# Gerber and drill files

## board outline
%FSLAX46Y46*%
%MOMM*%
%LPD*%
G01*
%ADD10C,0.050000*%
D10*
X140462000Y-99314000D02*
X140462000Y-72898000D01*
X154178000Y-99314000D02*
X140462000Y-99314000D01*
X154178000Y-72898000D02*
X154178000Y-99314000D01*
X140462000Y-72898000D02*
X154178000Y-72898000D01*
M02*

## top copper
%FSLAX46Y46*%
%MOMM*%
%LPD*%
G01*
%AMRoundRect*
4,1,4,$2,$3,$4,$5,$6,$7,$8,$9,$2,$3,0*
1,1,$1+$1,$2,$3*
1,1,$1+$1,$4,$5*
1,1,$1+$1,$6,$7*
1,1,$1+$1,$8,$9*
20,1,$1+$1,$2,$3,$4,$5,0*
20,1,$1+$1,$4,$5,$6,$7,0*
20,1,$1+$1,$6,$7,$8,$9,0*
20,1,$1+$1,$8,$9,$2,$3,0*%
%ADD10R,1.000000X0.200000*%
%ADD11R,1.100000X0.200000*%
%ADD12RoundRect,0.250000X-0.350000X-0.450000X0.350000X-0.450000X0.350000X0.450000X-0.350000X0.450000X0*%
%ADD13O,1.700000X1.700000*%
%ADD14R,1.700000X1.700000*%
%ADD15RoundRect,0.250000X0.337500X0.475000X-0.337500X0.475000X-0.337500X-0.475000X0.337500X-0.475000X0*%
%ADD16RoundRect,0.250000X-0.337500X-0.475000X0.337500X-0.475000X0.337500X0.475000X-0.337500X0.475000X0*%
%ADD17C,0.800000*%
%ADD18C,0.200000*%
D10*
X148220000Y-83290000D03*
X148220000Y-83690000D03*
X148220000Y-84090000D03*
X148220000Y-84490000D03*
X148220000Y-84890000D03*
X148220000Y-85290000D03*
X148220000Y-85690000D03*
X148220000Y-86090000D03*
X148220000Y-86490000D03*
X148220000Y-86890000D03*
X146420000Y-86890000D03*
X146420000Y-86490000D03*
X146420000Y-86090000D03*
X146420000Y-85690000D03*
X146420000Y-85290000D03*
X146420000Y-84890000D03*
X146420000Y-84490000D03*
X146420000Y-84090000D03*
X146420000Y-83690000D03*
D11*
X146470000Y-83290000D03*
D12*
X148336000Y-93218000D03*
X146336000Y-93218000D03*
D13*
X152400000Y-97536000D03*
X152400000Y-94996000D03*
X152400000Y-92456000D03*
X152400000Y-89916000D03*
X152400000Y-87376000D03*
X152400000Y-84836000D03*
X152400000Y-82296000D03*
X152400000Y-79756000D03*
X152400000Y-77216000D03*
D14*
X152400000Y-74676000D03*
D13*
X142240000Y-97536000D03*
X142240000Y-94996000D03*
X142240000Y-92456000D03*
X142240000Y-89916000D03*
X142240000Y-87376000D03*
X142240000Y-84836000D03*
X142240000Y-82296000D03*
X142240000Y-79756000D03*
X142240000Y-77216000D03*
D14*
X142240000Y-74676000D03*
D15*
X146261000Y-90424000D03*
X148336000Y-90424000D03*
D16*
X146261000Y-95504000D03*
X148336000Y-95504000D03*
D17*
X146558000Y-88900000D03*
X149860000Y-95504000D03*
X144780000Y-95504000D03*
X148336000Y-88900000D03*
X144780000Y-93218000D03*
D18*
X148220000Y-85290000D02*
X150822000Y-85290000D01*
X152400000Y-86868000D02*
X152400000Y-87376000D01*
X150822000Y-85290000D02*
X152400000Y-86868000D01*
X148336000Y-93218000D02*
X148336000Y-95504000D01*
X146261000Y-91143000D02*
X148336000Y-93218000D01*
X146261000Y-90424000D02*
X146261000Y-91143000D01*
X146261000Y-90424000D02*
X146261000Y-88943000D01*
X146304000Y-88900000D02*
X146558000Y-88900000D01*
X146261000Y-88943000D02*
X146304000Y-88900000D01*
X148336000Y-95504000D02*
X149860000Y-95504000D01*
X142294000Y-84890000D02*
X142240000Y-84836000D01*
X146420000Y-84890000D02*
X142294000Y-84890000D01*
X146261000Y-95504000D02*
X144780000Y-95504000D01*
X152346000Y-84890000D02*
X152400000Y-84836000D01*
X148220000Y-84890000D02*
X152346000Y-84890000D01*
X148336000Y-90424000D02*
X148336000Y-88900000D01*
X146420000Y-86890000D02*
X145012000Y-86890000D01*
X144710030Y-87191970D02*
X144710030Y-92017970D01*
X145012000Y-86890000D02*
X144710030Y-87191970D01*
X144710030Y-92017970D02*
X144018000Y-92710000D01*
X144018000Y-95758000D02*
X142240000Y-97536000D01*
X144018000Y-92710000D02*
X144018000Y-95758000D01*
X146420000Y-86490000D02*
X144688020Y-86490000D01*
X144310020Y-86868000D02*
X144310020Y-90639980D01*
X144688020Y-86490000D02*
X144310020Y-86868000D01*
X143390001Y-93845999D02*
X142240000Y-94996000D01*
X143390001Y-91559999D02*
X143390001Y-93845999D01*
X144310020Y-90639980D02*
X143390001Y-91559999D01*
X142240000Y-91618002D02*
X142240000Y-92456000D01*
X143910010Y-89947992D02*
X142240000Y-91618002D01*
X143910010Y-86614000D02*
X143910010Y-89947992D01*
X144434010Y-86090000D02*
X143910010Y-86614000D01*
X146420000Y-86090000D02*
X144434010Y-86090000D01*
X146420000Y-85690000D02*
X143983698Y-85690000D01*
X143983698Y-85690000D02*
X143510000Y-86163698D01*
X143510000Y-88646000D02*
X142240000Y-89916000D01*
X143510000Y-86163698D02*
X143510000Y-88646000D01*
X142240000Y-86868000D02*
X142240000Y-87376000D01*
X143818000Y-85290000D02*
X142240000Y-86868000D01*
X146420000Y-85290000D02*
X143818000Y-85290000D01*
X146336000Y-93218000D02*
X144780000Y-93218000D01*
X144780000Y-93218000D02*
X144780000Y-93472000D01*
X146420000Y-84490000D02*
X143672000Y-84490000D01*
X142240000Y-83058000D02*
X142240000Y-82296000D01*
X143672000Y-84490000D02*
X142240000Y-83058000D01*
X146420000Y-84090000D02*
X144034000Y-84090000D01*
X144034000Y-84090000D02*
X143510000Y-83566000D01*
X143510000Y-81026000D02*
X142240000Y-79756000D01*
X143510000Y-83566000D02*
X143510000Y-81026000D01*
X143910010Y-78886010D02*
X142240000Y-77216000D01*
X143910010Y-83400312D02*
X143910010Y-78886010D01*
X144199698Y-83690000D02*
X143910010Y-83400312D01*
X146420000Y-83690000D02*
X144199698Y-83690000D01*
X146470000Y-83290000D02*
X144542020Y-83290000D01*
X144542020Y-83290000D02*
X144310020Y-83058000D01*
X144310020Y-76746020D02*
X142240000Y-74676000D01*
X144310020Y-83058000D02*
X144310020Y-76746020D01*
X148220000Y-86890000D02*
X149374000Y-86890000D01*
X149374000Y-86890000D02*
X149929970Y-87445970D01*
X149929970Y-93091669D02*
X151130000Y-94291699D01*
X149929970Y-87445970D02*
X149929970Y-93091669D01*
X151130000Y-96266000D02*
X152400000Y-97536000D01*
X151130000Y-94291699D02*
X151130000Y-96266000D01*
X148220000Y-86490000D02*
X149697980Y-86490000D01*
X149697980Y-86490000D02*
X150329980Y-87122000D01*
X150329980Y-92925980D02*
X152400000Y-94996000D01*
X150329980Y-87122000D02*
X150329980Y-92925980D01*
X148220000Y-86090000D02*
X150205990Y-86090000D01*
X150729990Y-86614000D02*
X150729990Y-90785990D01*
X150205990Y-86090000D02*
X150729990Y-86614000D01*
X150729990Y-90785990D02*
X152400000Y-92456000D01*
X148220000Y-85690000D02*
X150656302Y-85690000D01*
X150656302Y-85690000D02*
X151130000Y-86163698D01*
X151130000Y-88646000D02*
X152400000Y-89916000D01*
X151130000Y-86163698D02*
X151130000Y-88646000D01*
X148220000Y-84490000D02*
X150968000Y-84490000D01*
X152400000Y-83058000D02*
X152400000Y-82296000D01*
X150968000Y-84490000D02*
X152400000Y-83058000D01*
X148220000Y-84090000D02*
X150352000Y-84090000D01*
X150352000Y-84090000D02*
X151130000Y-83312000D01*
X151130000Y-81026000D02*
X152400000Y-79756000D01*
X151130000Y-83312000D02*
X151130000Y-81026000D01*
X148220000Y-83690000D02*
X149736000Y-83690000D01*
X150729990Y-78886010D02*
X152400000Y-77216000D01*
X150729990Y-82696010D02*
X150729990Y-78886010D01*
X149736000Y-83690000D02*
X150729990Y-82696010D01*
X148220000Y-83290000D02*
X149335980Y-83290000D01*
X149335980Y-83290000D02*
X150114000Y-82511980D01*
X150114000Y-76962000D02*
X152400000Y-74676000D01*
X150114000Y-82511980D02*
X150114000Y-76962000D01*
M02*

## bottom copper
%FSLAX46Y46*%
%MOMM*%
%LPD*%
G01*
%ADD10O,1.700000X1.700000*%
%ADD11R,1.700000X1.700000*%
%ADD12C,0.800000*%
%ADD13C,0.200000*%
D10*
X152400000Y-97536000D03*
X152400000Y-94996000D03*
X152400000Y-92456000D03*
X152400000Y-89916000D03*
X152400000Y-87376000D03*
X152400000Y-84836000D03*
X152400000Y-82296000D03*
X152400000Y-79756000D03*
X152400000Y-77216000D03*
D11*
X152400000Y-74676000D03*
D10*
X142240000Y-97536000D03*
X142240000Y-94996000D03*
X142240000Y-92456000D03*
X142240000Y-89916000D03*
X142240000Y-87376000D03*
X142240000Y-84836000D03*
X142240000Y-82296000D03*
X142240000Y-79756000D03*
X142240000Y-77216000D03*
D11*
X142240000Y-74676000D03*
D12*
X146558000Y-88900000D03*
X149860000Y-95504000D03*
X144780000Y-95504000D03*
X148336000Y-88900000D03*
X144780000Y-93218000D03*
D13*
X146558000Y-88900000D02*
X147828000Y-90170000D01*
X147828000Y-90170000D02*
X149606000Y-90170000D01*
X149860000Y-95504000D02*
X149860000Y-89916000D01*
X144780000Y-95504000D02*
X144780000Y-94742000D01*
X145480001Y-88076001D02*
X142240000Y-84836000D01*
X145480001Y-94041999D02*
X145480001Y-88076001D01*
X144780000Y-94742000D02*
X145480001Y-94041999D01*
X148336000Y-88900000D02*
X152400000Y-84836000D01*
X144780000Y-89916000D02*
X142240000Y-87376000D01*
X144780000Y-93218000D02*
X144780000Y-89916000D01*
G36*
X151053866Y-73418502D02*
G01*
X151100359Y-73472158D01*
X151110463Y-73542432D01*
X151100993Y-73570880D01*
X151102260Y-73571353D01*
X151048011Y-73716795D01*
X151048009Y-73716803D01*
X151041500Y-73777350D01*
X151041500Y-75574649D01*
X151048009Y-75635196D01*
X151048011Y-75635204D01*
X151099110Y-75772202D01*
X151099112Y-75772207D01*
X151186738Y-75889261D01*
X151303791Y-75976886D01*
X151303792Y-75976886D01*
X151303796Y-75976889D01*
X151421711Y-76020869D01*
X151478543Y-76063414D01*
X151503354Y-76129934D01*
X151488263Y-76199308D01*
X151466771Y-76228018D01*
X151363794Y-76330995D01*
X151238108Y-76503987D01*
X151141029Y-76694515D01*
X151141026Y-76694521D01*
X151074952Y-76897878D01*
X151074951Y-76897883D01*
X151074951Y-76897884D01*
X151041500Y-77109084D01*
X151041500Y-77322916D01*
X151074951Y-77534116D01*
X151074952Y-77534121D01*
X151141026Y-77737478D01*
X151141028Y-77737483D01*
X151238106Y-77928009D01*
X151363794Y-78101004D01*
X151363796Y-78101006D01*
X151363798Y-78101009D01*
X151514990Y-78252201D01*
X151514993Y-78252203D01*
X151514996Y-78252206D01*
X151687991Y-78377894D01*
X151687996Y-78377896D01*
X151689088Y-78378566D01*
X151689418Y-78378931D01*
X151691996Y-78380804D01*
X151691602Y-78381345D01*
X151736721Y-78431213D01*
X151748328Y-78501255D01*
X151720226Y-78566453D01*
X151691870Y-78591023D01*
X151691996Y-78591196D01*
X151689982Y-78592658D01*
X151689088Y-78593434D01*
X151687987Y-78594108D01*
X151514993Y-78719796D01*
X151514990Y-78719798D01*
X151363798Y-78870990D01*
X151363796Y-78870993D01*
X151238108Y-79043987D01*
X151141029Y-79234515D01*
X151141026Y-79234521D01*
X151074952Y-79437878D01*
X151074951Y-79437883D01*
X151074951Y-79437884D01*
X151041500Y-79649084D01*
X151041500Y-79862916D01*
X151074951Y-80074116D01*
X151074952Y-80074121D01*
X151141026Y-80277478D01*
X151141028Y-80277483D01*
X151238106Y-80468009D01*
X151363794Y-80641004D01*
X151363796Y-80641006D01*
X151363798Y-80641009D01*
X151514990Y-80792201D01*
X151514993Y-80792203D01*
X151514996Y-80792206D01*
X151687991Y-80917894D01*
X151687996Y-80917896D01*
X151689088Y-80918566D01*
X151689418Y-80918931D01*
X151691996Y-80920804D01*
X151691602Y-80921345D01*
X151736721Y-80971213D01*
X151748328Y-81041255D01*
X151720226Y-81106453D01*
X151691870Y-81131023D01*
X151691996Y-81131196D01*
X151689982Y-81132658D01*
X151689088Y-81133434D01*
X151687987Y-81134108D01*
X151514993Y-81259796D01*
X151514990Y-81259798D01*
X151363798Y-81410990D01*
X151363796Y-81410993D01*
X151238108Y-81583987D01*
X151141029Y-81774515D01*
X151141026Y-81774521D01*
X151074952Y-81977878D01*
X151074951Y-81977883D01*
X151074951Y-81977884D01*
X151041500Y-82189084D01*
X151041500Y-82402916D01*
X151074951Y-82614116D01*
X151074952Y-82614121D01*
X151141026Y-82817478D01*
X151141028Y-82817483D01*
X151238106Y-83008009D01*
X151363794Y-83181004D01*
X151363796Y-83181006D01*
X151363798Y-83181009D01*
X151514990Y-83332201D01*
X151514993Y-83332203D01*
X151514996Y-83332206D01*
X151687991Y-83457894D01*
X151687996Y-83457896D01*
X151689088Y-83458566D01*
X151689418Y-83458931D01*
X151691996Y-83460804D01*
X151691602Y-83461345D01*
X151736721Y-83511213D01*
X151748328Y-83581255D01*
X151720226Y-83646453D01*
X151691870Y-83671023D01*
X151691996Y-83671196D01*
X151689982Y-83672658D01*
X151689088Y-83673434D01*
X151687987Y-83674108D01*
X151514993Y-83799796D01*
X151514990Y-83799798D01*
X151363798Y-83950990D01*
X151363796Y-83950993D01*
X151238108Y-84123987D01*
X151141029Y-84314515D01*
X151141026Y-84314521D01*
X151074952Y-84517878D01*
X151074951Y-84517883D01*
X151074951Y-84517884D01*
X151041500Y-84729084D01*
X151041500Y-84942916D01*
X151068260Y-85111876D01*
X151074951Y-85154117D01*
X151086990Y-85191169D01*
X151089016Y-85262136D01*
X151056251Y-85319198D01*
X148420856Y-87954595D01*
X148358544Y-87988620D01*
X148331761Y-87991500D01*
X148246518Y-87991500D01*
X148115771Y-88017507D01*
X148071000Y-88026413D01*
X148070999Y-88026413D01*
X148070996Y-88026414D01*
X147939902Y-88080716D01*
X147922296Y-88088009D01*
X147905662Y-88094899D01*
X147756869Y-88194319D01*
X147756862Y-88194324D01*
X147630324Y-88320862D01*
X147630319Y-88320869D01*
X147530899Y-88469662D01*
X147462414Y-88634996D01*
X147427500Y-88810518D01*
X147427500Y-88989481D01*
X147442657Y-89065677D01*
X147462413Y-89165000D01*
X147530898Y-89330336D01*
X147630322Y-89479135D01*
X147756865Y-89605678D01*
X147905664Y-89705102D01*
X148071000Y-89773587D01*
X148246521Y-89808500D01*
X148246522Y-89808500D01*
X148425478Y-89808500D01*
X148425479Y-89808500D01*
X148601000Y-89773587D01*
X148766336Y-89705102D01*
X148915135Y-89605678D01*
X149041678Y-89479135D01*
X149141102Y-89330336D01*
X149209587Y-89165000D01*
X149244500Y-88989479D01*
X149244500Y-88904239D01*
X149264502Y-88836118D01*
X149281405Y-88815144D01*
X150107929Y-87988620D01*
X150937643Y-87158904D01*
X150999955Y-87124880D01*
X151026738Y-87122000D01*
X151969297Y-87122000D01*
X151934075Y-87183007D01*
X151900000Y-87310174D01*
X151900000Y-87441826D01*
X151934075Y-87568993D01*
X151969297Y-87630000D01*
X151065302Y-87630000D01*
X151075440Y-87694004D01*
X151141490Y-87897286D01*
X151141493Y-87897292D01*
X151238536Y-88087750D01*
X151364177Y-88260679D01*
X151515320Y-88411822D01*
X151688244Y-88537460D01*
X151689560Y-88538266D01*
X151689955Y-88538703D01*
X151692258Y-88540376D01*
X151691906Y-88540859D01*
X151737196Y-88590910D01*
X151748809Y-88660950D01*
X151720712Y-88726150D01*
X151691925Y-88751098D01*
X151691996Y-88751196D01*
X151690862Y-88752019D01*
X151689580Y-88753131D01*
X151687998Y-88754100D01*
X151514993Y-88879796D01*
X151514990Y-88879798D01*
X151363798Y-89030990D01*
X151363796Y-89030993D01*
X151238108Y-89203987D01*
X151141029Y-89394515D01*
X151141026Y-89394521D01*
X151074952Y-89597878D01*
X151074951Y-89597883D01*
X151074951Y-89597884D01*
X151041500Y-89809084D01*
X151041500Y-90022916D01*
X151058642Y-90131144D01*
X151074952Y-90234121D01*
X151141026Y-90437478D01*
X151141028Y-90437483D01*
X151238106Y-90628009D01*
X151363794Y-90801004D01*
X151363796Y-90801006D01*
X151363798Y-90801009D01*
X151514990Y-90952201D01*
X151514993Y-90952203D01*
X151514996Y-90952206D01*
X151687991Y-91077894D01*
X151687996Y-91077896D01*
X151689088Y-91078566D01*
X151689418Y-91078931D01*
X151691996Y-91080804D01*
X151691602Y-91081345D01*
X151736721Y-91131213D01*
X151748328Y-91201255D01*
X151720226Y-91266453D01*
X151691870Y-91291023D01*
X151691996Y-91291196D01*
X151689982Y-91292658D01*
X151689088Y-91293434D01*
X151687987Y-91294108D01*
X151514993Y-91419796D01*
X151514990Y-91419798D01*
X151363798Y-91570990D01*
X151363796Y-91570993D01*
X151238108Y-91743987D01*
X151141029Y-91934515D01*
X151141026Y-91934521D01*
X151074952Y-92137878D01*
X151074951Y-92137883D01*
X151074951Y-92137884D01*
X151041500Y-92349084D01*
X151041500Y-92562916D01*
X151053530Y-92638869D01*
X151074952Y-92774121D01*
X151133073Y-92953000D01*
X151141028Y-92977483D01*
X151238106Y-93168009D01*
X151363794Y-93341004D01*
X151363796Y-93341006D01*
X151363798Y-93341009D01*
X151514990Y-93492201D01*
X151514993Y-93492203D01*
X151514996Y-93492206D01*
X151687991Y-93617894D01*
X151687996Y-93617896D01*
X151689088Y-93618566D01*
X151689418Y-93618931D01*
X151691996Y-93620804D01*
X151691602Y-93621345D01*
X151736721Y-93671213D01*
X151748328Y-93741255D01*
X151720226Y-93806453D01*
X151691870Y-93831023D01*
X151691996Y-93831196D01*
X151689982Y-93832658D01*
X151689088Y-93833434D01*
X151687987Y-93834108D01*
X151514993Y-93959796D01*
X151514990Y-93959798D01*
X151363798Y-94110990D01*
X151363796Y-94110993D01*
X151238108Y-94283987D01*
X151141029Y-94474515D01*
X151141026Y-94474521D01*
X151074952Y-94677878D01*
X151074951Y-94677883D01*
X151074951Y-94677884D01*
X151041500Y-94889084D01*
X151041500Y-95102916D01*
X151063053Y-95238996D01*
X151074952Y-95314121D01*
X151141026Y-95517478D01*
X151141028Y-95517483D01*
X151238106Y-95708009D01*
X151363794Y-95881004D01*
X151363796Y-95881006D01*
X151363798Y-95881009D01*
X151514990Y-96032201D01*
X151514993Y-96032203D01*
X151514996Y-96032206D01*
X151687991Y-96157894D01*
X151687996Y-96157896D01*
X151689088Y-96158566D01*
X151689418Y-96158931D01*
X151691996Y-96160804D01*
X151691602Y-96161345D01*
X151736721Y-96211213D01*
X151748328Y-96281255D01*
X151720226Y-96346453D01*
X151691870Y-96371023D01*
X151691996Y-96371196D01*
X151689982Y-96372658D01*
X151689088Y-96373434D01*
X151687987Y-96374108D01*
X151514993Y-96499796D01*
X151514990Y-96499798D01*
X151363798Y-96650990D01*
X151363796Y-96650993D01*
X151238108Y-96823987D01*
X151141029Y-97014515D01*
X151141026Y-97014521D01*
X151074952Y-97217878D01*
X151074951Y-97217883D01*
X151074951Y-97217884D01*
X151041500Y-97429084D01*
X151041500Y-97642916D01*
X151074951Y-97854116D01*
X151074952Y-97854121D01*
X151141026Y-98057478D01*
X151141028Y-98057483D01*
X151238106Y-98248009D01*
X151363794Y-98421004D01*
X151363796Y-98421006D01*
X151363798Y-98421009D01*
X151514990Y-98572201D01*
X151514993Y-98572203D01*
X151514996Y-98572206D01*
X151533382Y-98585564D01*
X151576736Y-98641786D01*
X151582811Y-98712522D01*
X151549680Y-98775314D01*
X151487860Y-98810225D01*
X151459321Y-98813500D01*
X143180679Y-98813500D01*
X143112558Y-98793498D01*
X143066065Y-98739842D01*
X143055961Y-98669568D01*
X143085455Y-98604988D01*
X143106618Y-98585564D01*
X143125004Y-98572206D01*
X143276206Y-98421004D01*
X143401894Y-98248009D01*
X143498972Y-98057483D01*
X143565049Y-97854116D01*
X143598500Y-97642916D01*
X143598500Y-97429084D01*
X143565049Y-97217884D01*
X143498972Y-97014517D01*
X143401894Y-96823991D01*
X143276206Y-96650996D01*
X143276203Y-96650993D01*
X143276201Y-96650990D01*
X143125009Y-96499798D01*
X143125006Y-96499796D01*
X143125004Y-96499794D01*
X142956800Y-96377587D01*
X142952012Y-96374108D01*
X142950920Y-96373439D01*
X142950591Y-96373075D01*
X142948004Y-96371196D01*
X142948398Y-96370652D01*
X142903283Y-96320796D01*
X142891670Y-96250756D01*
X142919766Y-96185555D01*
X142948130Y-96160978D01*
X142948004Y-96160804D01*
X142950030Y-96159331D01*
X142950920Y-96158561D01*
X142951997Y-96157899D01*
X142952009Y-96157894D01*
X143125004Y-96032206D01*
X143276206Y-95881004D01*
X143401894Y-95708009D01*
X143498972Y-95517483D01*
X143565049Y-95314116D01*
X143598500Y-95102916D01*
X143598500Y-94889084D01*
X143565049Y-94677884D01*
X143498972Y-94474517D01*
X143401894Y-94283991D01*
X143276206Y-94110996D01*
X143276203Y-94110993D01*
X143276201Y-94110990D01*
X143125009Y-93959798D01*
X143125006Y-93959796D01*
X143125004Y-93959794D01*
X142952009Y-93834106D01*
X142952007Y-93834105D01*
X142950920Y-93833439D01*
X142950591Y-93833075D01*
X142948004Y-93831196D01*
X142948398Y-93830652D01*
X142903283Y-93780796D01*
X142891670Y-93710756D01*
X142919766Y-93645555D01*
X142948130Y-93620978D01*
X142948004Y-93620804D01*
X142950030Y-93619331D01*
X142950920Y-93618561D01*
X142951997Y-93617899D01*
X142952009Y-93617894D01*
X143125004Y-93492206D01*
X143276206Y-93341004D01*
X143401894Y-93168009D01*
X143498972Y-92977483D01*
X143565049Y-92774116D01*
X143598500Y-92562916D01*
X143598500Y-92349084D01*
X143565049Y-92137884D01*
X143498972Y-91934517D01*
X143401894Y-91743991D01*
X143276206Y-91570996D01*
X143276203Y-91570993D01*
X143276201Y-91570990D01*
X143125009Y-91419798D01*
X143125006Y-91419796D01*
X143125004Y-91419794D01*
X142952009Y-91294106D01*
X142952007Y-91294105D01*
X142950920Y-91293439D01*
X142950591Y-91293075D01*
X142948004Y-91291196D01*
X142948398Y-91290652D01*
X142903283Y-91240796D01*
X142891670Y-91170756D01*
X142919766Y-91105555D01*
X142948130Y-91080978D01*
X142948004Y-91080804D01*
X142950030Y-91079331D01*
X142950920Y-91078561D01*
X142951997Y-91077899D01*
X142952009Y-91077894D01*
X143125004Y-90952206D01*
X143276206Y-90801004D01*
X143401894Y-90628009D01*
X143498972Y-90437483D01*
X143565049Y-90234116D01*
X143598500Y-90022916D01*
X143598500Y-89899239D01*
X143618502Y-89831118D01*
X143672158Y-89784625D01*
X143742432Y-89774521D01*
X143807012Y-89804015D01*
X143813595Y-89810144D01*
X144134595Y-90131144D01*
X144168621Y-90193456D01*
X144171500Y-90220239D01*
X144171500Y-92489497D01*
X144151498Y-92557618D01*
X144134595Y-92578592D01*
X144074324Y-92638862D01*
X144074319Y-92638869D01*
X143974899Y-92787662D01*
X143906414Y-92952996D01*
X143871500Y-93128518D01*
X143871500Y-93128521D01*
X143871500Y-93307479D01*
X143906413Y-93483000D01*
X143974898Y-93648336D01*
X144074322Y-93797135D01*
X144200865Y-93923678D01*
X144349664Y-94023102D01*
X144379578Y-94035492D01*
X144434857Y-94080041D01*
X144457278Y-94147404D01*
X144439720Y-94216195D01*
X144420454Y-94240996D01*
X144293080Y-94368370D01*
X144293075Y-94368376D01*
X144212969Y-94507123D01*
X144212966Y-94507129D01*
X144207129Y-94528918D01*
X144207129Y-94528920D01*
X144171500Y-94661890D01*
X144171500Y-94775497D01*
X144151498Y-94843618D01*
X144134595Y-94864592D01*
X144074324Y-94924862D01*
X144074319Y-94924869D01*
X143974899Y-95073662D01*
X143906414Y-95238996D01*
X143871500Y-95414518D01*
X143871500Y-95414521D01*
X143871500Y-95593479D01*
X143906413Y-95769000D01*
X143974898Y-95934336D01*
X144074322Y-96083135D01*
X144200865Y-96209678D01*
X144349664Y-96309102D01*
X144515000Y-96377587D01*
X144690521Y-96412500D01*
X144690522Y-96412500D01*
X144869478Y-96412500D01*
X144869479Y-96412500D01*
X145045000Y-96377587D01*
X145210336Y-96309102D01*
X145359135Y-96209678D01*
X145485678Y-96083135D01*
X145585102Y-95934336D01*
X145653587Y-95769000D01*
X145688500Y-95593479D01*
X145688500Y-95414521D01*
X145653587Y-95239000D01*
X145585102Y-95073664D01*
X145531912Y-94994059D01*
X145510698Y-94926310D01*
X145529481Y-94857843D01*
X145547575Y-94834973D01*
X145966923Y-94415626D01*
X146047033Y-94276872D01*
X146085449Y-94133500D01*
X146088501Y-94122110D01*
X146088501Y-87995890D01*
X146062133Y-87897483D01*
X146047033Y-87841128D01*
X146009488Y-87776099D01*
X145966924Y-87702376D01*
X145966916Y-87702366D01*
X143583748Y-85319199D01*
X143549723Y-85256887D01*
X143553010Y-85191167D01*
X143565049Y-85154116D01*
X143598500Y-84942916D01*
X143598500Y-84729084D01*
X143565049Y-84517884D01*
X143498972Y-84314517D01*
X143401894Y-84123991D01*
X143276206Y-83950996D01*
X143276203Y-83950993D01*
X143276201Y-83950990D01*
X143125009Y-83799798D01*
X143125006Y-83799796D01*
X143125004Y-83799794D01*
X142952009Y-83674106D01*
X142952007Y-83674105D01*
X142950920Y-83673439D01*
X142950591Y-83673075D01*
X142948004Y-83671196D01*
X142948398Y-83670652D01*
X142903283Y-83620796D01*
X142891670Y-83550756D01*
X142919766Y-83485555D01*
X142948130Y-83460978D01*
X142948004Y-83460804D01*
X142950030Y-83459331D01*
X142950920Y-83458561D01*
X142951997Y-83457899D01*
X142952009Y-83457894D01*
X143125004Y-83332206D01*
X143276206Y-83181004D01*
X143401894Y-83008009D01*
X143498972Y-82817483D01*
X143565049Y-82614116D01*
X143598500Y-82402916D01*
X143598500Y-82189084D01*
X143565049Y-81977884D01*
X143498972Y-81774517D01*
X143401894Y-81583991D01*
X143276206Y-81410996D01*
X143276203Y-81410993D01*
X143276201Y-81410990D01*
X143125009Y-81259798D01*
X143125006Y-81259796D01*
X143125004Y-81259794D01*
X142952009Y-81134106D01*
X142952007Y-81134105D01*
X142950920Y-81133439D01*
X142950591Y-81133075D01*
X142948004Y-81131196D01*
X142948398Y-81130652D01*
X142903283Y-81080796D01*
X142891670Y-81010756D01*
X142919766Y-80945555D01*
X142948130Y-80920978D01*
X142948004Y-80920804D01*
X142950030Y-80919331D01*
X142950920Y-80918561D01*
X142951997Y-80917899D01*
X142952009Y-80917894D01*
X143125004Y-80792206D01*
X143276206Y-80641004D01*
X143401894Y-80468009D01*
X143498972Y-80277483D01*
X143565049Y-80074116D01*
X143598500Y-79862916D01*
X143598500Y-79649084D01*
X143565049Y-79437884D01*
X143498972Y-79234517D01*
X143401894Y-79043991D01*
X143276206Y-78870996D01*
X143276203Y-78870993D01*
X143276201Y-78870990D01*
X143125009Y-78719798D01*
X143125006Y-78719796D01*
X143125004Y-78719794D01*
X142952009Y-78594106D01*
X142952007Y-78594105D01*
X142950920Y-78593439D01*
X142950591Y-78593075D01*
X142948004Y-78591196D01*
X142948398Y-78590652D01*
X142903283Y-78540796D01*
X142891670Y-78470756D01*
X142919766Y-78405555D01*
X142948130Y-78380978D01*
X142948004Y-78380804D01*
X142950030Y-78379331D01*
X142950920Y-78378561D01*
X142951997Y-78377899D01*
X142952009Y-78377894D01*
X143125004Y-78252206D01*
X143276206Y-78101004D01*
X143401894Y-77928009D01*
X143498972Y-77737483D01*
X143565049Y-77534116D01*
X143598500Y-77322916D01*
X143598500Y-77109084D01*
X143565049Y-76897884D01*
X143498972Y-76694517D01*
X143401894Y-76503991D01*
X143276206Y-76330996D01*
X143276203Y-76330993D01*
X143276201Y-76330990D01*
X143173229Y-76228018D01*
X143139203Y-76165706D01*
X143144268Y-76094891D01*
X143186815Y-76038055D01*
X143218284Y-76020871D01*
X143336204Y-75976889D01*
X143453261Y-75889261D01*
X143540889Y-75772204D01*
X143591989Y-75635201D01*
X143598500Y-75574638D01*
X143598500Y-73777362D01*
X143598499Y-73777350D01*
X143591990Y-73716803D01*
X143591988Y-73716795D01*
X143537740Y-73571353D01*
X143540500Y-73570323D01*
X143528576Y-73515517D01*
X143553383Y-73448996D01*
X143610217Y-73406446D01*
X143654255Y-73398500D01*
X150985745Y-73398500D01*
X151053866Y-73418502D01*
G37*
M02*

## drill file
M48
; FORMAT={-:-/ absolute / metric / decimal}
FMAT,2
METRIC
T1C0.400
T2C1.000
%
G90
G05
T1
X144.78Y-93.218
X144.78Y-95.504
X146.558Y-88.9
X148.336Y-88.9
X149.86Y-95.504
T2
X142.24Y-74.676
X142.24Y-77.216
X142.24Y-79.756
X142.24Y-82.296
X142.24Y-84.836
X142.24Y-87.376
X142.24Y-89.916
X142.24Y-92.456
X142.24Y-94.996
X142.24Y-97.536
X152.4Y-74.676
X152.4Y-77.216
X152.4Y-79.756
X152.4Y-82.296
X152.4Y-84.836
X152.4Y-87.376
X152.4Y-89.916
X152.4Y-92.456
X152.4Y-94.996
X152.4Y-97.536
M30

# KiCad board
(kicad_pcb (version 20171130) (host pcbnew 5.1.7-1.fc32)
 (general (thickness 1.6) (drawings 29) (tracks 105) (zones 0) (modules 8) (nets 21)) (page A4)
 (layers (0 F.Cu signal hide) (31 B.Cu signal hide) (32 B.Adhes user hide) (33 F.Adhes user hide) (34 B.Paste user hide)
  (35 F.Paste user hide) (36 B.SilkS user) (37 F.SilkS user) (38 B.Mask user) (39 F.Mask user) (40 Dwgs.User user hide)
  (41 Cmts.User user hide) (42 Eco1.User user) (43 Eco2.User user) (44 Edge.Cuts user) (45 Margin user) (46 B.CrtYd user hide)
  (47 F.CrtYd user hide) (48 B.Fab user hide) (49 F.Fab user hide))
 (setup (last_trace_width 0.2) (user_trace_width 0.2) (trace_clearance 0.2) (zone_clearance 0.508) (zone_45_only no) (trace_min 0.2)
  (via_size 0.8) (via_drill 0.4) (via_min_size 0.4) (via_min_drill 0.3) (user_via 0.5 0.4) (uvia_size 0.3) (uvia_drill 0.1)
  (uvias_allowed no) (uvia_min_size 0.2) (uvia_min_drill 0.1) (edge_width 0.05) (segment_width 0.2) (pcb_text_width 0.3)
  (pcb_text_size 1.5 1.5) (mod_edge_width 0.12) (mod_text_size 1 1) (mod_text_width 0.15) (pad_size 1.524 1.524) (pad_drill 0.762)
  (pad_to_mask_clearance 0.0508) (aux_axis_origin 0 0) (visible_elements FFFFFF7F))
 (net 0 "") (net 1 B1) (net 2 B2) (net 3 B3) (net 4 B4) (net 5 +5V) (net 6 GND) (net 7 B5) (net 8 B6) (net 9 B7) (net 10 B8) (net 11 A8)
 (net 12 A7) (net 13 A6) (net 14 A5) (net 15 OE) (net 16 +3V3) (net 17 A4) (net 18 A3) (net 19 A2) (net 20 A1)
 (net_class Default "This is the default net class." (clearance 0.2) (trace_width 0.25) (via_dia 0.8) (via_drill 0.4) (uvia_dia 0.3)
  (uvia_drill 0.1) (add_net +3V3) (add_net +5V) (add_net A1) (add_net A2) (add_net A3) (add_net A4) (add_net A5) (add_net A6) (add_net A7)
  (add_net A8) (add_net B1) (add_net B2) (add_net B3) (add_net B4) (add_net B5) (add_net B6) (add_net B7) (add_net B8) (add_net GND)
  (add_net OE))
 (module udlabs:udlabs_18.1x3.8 (layer B.Cu) (at 147.5232 85.598 90)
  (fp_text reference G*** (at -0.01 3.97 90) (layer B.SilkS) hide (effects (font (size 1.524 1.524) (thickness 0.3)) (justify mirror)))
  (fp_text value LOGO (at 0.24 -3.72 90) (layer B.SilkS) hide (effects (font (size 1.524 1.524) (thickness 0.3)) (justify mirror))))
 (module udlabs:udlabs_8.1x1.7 (layer F.Cu) (at 147.066 77.7494 90)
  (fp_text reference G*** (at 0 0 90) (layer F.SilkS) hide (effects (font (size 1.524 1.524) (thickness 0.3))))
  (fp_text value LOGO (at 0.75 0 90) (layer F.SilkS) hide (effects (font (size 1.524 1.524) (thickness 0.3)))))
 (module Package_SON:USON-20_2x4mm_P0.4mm (layer F.Cu) (at 147.32 85.09)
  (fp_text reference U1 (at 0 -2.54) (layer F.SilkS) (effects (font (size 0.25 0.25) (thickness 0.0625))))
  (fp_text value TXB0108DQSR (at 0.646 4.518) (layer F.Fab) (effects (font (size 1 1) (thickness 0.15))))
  (pad 20 smd rect (at 0.9 -1.8 270) (size 0.2 1) (layers F.Cu F.Paste F.Mask) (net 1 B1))
  (pad 19 smd rect (at 0.9 -1.4 270) (size 0.2 1) (layers F.Cu F.Paste F.Mask) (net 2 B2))
  (pad 18 smd rect (at 0.9 -1 270) (size 0.2 1) (layers F.Cu F.Paste F.Mask) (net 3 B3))
  (pad 17 smd rect (at 0.9 -0.6 270) (size 0.2 1) (layers F.Cu F.Paste F.Mask) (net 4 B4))
  (pad 16 smd rect (at 0.9 -0.2 270) (size 0.2 1) (layers F.Cu F.Paste F.Mask) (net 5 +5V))
  (pad 15 smd rect (at 0.9 0.2 270) (size 0.2 1) (layers F.Cu F.Paste F.Mask) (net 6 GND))
  (pad 14 smd rect (at 0.9 0.6 270) (size 0.2 1) (layers F.Cu F.Paste F.Mask) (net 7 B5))
  (pad 13 smd rect (at 0.9 1 270) (size 0.2 1) (layers F.Cu F.Paste F.Mask) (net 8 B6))
  (pad 12 smd rect (at 0.9 1.4 270) (size 0.2 1) (layers F.Cu F.Paste F.Mask) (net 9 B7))
  (pad 11 smd rect (at 0.9 1.8 270) (size 0.2 1) (layers F.Cu F.Paste F.Mask) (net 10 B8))
  (pad 10 smd rect (at -0.9 1.8 270) (size 0.2 1) (layers F.Cu F.Paste F.Mask) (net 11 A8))
  (pad 9 smd rect (at -0.9 1.4 270) (size 0.2 1) (layers F.Cu F.Paste F.Mask) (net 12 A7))
  (pad 8 smd rect (at -0.9 1 270) (size 0.2 1) (layers F.Cu F.Paste F.Mask) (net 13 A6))
  (pad 7 smd rect (at -0.9 0.6 270) (size 0.2 1) (layers F.Cu F.Paste F.Mask) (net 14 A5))
  (pad 6 smd rect (at -0.9 0.2 270) (size 0.2 1) (layers F.Cu F.Paste F.Mask) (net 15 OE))
  (pad 5 smd rect (at -0.9 -0.2 270) (size 0.2 1) (layers F.Cu F.Paste F.Mask) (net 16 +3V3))
  (pad 4 smd rect (at -0.9 -0.6 270) (size 0.2 1) (layers F.Cu F.Paste F.Mask) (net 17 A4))
  (pad 3 smd rect (at -0.9 -1 270) (size 0.2 1) (layers F.Cu F.Paste F.Mask) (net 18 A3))
  (pad 2 smd rect (at -0.9 -1.4 270) (size 0.2 1) (layers F.Cu F.Paste F.Mask) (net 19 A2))
  (pad 1 smd rect (at -0.85 -1.8 270) (size 0.2 1.1) (layers F.Cu F.Paste F.Mask) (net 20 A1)))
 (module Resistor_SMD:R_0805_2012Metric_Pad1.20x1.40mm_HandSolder (layer F.Cu) (at 147.336 93.218)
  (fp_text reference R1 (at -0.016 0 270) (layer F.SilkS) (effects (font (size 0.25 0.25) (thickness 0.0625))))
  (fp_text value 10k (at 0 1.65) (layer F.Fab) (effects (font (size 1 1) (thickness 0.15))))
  (pad 2 smd roundrect (at 1 0) (size 1.2 1.4) (layers F.Cu F.Paste F.Mask) (roundrect_rratio 0.208333) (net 6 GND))
  (pad 1 smd roundrect (at -1 0) (size 1.2 1.4) (layers F.Cu F.Paste F.Mask) (roundrect_rratio 0.208333) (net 15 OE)))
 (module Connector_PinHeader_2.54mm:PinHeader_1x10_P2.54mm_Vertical (layer B.Cu) (at 152.4 74.676 180)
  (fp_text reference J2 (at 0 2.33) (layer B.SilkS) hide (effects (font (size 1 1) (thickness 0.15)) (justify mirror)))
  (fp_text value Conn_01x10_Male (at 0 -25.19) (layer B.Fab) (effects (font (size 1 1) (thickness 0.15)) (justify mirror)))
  (pad 10 thru_hole oval (at 0 -22.86 180) (size 1.7 1.7) (drill 1) (layers *.Cu *.Mask) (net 10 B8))
  (pad 9 thru_hole oval (at 0 -20.32 180) (size 1.7 1.7) (drill 1) (layers *.Cu *.Mask) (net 9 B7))
  (pad 8 thru_hole oval (at 0 -17.78 180) (size 1.7 1.7) (drill 1) (layers *.Cu *.Mask) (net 8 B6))
  (pad 7 thru_hole oval (at 0 -15.24 180) (size 1.7 1.7) (drill 1) (layers *.Cu *.Mask) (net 7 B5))
  (pad 6 thru_hole oval (at 0 -12.7 180) (size 1.7 1.7) (drill 1) (layers *.Cu *.Mask) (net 6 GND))
  (pad 5 thru_hole oval (at 0 -10.16 180) (size 1.7 1.7) (drill 1) (layers *.Cu *.Mask) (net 5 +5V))
  (pad 4 thru_hole oval (at 0 -7.62 180) (size 1.7 1.7) (drill 1) (layers *.Cu *.Mask) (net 4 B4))
  (pad 3 thru_hole oval (at 0 -5.08 180) (size 1.7 1.7) (drill 1) (layers *.Cu *.Mask) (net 3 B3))
  (pad 2 thru_hole oval (at 0 -2.54 180) (size 1.7 1.7) (drill 1) (layers *.Cu *.Mask) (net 2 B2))
  (pad 1 thru_hole rect (at 0 0 180) (size 1.7 1.7) (drill 1) (layers *.Cu *.Mask) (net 1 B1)))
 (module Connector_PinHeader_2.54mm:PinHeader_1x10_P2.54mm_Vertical (layer B.Cu) (at 142.24 74.676 180)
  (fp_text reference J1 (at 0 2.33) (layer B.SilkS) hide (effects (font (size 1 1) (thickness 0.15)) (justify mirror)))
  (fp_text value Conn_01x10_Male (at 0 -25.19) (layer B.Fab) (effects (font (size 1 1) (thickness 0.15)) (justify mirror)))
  (pad 10 thru_hole oval (at 0 -22.86 180) (size 1.7 1.7) (drill 1) (layers *.Cu *.Mask) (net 11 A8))
  (pad 9 thru_hole oval (at 0 -20.32 180) (size 1.7 1.7) (drill 1) (layers *.Cu *.Mask) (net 12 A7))
  (pad 8 thru_hole oval (at 0 -17.78 180) (size 1.7 1.7) (drill 1) (layers *.Cu *.Mask) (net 13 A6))
  (pad 7 thru_hole oval (at 0 -15.24 180) (size 1.7 1.7) (drill 1) (layers *.Cu *.Mask) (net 14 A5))
  (pad 6 thru_hole oval (at 0 -12.7 180) (size 1.7 1.7) (drill 1) (layers *.Cu *.Mask) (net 15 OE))
  (pad 5 thru_hole oval (at 0 -10.16 180) (size 1.7 1.7) (drill 1) (layers *.Cu *.Mask) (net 16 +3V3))
  (pad 4 thru_hole oval (at 0 -7.62 180) (size 1.7 1.7) (drill 1) (layers *.Cu *.Mask) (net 17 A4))
  (pad 3 thru_hole oval (at 0 -5.08 180) (size 1.7 1.7) (drill 1) (layers *.Cu *.Mask) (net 18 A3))
  (pad 2 thru_hole oval (at 0 -2.54 180) (size 1.7 1.7) (drill 1) (layers *.Cu *.Mask) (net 19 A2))
  (pad 1 thru_hole rect (at 0 0 180) (size 1.7 1.7) (drill 1) (layers *.Cu *.Mask) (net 20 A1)))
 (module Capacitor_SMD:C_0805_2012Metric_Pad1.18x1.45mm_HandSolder (layer F.Cu) (at 147.2985 90.424 180)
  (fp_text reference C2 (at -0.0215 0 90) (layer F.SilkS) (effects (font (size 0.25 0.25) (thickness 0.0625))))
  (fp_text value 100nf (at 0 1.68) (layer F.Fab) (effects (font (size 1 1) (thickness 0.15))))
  (pad 2 smd roundrect (at 1.0375 0 180) (size 1.175 1.45) (layers F.Cu F.Paste F.Mask) (roundrect_rratio 0.212766) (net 6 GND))
  (pad 1 smd roundrect (at -1.0375 0 180) (size 1.175 1.45) (layers F.Cu F.Paste F.Mask) (roundrect_rratio 0.212766) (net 5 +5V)))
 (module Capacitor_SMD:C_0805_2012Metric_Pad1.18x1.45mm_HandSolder (layer F.Cu) (at 147.2985 95.504)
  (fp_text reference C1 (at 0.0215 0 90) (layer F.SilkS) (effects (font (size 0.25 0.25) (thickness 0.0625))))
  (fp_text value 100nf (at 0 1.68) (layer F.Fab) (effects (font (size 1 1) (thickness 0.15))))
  (pad 1 smd roundrect (at -1.0375 0) (size 1.175 1.45) (layers F.Cu F.Paste F.Mask) (roundrect_rratio 0.212766) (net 16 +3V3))
  (pad 2 smd roundrect (at 1.0375 0) (size 1.175 1.45) (layers F.Cu F.Paste F.Mask) (roundrect_rratio 0.212766) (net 6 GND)))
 (gr_line (start 140.462 99.314) (end 140.462 72.898) (layer Edge.Cuts) (width 0.05))
 (gr_line (start 154.178 99.314) (end 140.462 99.314) (layer Edge.Cuts) (width 0.05))
 (gr_line (start 154.178 72.898) (end 154.178 99.314) (layer Edge.Cuts) (width 0.05))
 (gr_line (start 140.462 72.898) (end 154.178 72.898) (layer Edge.Cuts) (width 0.05))
 (segment (start 148.22 85.29) (end 150.822 85.29) (width 0.2) (layer F.Cu) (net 6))
 (segment (start 152.4 86.868) (end 152.4 87.376) (width 0.2) (layer F.Cu) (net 6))
 (segment (start 150.822 85.29) (end 152.4 86.868) (width 0.2) (layer F.Cu) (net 6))
 (segment (start 148.336 93.218) (end 148.336 95.504) (width 0.2) (layer F.Cu) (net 6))
 (segment (start 146.261 91.143) (end 148.336 93.218) (width 0.2) (layer F.Cu) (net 6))
 (segment (start 146.261 90.424) (end 146.261 91.143) (width 0.2) (layer F.Cu) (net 6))
 (segment (start 146.261 90.424) (end 146.261 88.943) (width 0.2) (layer F.Cu) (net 6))
 (via (at 146.558 88.9) (size 0.8) (drill 0.4) (layers F.Cu B.Cu) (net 6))
 (segment (start 146.304 88.9) (end 146.558 88.9) (width 0.2) (layer F.Cu) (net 6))
 (segment (start 146.261 88.943) (end 146.304 88.9) (width 0.2) (layer F.Cu) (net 6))
 (segment (start 146.558 88.9) (end 147.828 90.17) (width 0.2) (layer B.Cu) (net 6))
 (segment (start 147.828 90.17) (end 149.606 90.17) (width 0.2) (layer B.Cu) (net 6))
 (segment (start 148.336 95.504) (end 149.86 95.504) (width 0.2) (layer F.Cu) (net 6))
 (via (at 149.86 95.504) (size 0.8) (drill 0.4) (layers F.Cu B.Cu) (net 6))
 (segment (start 149.86 95.504) (end 149.86 89.916) (width 0.2) (layer B.Cu) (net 6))
 (segment (start 142.294 84.89) (end 142.24 84.836) (width 0.2) (layer F.Cu) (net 16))
 (segment (start 146.42 84.89) (end 142.294 84.89) (width 0.2) (layer F.Cu) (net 16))
 (segment (start 146.261 95.504) (end 144.78 95.504) (width 0.2) (layer F.Cu) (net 16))
 (via (at 144.78 95.504) (size 0.8) (drill 0.4) (layers F.Cu B.Cu) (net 16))
 (segment (start 144.78 95.504) (end 144.78 94.742) (width 0.2) (layer B.Cu) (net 16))
 (segment (start 145.480001 88.076001) (end 142.24 84.836) (width 0.2) (layer B.Cu) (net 16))
 (segment (start 145.480001 94.041999) (end 145.480001 88.076001) (width 0.2) (layer B.Cu) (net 16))
 (segment (start 144.78 94.742) (end 145.480001 94.041999) (width 0.2) (layer B.Cu) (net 16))
 (segment (start 152.346 84.89) (end 152.4 84.836) (width 0.2) (layer F.Cu) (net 5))
 (segment (start 148.22 84.89) (end 152.346 84.89) (width 0.2) (layer F.Cu) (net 5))
 (segment (start 148.336 90.424) (end 148.336 88.9) (width 0.2) (layer F.Cu) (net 5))
 (via (at 148.336 88.9) (size 0.8) (drill 0.4) (layers F.Cu B.Cu) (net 5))
 (segment (start 148.336 88.9) (end 152.4 84.836) (width 0.2) (layer B.Cu) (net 5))
 (segment (start 146.42 86.89) (end 145.012 86.89) (width 0.2) (layer F.Cu) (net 11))
 (segment (start 144.71003 87.19197) (end 144.71003 92.01797) (width 0.2) (layer F.Cu) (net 11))
 (segment (start 145.012 86.89) (end 144.71003 87.19197) (width 0.2) (layer F.Cu) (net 11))
 (segment (start 144.71003 92.01797) (end 144.018 92.71) (width 0.2) (layer F.Cu) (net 11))
 (segment (start 144.018 95.758) (end 142.24 97.536) (width 0.2) (layer F.Cu) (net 11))
 (segment (start 144.018 92.71) (end 144.018 95.758) (width 0.2) (layer F.Cu) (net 11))
 (segment (start 146.42 86.49) (end 144.68802 86.49) (width 0.2) (layer F.Cu) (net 12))
 (segment (start 144.31002 86.868) (end 144.31002 90.63998) (width 0.2) (layer F.Cu) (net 12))
 (segment (start 144.68802 86.49) (end 144.31002 86.868) (width 0.2) (layer F.Cu) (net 12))
 (segment (start 143.390001 93.845999) (end 142.24 94.996) (width 0.2) (layer F.Cu) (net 12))
 (segment (start 143.390001 91.559999) (end 143.390001 93.845999) (width 0.2) (layer F.Cu) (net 12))
 (segment (start 144.31002 90.63998) (end 143.390001 91.559999) (width 0.2) (layer F.Cu) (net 12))
 (segment (start 142.24 91.618002) (end 142.24 92.456) (width 0.2) (layer F.Cu) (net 13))
 (segment (start 143.91001 89.947992) (end 142.24 91.618002) (width 0.2) (layer F.Cu) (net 13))
 (segment (start 143.91001 86.614) (end 143.91001 89.947992) (width 0.2) (layer F.Cu) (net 13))
 (segment (start 144.43401 86.09) (end 143.91001 86.614) (width 0.2) (layer F.Cu) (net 13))
 (segment (start 146.42 86.09) (end 144.43401 86.09) (width 0.2) (layer F.Cu) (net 13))
 (segment (start 146.42 85.69) (end 143.983698 85.69) (width 0.2) (layer F.Cu) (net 14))
 (segment (start 143.983698 85.69) (end 143.51 86.163698) (width 0.2) (layer F.Cu) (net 14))
 (segment (start 143.51 88.646) (end 142.24 89.916) (width 0.2) (layer F.Cu) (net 14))
 (segment (start 143.51 86.163698) (end 143.51 88.646) (width 0.2) (layer F.Cu) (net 14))
 (segment (start 142.24 86.868) (end 142.24 87.376) (width 0.2) (layer F.Cu) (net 15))
 (segment (start 143.818 85.29) (end 142.24 86.868) (width 0.2) (layer F.Cu) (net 15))
 (segment (start 146.42 85.29) (end 143.818 85.29) (width 0.2) (layer F.Cu) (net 15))
 (segment (start 146.336 93.218) (end 144.78 93.218) (width 0.2) (layer F.Cu) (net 15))
 (via (at 144.78 93.218) (size 0.8) (drill 0.4) (layers F.Cu B.Cu) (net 15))
 (segment (start 144.78 93.218) (end 144.78 93.472) (width 0.2) (layer F.Cu) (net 15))
 (segment (start 144.78 89.916) (end 142.24 87.376) (width 0.2) (layer B.Cu) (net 15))
 (segment (start 144.78 93.218) (end 144.78 89.916) (width 0.2) (layer B.Cu) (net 15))
 (segment (start 146.42 84.49) (end 143.672 84.49) (width 0.2) (layer F.Cu) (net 17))
 (segment (start 142.24 83.058) (end 142.24 82.296) (width 0.2) (layer F.Cu) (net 17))
 (segment (start 143.672 84.49) (end 142.24 83.058) (width 0.2) (layer F.Cu) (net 17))
 (segment (start 146.42 84.09) (end 144.034 84.09) (width 0.2) (layer F.Cu) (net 18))
 (segment (start 144.034 84.09) (end 143.51 83.566) (width 0.2) (layer F.Cu) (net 18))
 (segment (start 143.51 81.026) (end 142.24 79.756) (width 0.2) (layer F.Cu) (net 18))
 (segment (start 143.51 83.566) (end 143.51 81.026) (width 0.2) (layer F.Cu) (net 18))
 (segment (start 143.91001 78.88601) (end 142.24 77.216) (width 0.2) (layer F.Cu) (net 19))
 (segment (start 143.91001 83.400312) (end 143.91001 78.88601) (width 0.2) (layer F.Cu) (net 19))
 (segment (start 144.199698 83.69) (end 143.91001 83.400312) (width 0.2) (layer F.Cu) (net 19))
 (segment (start 146.42 83.69) (end 144.199698 83.69) (width 0.2) (layer F.Cu) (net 19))
 (segment (start 146.47 83.29) (end 144.54202 83.29) (width 0.2) (layer F.Cu) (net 20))
 (segment (start 144.54202 83.29) (end 144.31002 83.058) (width 0.2) (layer F.Cu) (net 20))
 (segment (start 144.31002 76.74602) (end 142.24 74.676) (width 0.2) (layer F.Cu) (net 20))
 (segment (start 144.31002 83.058) (end 144.31002 76.74602) (width 0.2) (layer F.Cu) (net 20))
 (segment (start 148.22 86.89) (end 149.374 86.89) (width 0.2) (layer F.Cu) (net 10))
 (segment (start 149.374 86.89) (end 149.92997 87.44597) (width 0.2) (layer F.Cu) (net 10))
 (segment (start 149.92997 93.091669) (end 151.13 94.291699) (width 0.2) (layer F.Cu) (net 10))
 (segment (start 149.92997 87.44597) (end 149.92997 93.091669) (width 0.2) (layer F.Cu) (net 10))
 (segment (start 151.13 96.266) (end 152.4 97.536) (width 0.2) (layer F.Cu) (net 10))
 (segment (start 151.13 94.291699) (end 151.13 96.266) (width 0.2) (layer F.Cu) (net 10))
 (segment (start 148.22 86.49) (end 149.69798 86.49) (width 0.2) (layer F.Cu) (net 9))
 (segment (start 149.69798 86.49) (end 150.32998 87.122) (width 0.2) (layer F.Cu) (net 9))
 (segment (start 150.32998 92.92598) (end 152.4 94.996) (width 0.2) (layer F.Cu) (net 9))
 (segment (start 150.32998 87.122) (end 150.32998 92.92598) (width 0.2) (layer F.Cu) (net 9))
 (segment (start 148.22 86.09) (end 150.20599 86.09) (width 0.2) (layer F.Cu) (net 8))
 (segment (start 150.72999 86.614) (end 150.72999 90.78599) (width 0.2) (layer F.Cu) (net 8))
 (segment (start 150.20599 86.09) (end 150.72999 86.614) (width 0.2) (layer F.Cu) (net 8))
 (segment (start 150.72999 90.78599) (end 152.4 92.456) (width 0.2) (layer F.Cu) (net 8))
 (segment (start 148.22 85.69) (end 150.656302 85.69) (width 0.2) (layer F.Cu) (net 7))
 (segment (start 150.656302 85.69) (end 151.13 86.163698) (width 0.2) (layer F.Cu) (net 7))
 (segment (start 151.13 88.646) (end 152.4 89.916) (width 0.2) (layer F.Cu) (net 7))
 (segment (start 151.13 86.163698) (end 151.13 88.646) (width 0.2) (layer F.Cu) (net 7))
 (segment (start 148.22 84.49) (end 150.968 84.49) (width 0.2) (layer F.Cu) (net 4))
 (segment (start 152.4 83.058) (end 152.4 82.296) (width 0.2) (layer F.Cu) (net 4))
 (segment (start 150.968 84.49) (end 152.4 83.058) (width 0.2) (layer F.Cu) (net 4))
 (segment (start 148.22 84.09) (end 150.352 84.09) (width 0.2) (layer F.Cu) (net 3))
 (segment (start 150.352 84.09) (end 151.13 83.312) (width 0.2) (layer F.Cu) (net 3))
 (segment (start 151.13 81.026) (end 152.4 79.756) (width 0.2) (layer F.Cu) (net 3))
 (segment (start 151.13 83.312) (end 151.13 81.026) (width 0.2) (layer F.Cu) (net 3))
 (segment (start 148.22 83.69) (end 149.736 83.69) (width 0.2) (layer F.Cu) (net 2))
 (segment (start 150.72999 78.88601) (end 152.4 77.216) (width 0.2) (layer F.Cu) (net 2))
 (segment (start 150.72999 82.69601) (end 150.72999 78.88601) (width 0.2) (layer F.Cu) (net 2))
 (segment (start 149.736 83.69) (end 150.72999 82.69601) (width 0.2) (layer F.Cu) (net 2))
 (segment (start 148.22 83.29) (end 149.33598 83.29) (width 0.2) (layer F.Cu) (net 1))
 (segment (start 149.33598 83.29) (end 150.114 82.51198) (width 0.2) (layer F.Cu) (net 1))
 (segment (start 150.114 76.962) (end 152.4 74.676) (width 0.2) (layer F.Cu) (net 1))
 (segment (start 150.114 82.51198) (end 150.114 76.962) (width 0.2) (layer F.Cu) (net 1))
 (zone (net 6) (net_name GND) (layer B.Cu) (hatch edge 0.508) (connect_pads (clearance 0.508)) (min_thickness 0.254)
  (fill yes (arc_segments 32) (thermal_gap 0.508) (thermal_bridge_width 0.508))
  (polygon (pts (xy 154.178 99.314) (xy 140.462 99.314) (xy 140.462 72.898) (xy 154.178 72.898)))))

